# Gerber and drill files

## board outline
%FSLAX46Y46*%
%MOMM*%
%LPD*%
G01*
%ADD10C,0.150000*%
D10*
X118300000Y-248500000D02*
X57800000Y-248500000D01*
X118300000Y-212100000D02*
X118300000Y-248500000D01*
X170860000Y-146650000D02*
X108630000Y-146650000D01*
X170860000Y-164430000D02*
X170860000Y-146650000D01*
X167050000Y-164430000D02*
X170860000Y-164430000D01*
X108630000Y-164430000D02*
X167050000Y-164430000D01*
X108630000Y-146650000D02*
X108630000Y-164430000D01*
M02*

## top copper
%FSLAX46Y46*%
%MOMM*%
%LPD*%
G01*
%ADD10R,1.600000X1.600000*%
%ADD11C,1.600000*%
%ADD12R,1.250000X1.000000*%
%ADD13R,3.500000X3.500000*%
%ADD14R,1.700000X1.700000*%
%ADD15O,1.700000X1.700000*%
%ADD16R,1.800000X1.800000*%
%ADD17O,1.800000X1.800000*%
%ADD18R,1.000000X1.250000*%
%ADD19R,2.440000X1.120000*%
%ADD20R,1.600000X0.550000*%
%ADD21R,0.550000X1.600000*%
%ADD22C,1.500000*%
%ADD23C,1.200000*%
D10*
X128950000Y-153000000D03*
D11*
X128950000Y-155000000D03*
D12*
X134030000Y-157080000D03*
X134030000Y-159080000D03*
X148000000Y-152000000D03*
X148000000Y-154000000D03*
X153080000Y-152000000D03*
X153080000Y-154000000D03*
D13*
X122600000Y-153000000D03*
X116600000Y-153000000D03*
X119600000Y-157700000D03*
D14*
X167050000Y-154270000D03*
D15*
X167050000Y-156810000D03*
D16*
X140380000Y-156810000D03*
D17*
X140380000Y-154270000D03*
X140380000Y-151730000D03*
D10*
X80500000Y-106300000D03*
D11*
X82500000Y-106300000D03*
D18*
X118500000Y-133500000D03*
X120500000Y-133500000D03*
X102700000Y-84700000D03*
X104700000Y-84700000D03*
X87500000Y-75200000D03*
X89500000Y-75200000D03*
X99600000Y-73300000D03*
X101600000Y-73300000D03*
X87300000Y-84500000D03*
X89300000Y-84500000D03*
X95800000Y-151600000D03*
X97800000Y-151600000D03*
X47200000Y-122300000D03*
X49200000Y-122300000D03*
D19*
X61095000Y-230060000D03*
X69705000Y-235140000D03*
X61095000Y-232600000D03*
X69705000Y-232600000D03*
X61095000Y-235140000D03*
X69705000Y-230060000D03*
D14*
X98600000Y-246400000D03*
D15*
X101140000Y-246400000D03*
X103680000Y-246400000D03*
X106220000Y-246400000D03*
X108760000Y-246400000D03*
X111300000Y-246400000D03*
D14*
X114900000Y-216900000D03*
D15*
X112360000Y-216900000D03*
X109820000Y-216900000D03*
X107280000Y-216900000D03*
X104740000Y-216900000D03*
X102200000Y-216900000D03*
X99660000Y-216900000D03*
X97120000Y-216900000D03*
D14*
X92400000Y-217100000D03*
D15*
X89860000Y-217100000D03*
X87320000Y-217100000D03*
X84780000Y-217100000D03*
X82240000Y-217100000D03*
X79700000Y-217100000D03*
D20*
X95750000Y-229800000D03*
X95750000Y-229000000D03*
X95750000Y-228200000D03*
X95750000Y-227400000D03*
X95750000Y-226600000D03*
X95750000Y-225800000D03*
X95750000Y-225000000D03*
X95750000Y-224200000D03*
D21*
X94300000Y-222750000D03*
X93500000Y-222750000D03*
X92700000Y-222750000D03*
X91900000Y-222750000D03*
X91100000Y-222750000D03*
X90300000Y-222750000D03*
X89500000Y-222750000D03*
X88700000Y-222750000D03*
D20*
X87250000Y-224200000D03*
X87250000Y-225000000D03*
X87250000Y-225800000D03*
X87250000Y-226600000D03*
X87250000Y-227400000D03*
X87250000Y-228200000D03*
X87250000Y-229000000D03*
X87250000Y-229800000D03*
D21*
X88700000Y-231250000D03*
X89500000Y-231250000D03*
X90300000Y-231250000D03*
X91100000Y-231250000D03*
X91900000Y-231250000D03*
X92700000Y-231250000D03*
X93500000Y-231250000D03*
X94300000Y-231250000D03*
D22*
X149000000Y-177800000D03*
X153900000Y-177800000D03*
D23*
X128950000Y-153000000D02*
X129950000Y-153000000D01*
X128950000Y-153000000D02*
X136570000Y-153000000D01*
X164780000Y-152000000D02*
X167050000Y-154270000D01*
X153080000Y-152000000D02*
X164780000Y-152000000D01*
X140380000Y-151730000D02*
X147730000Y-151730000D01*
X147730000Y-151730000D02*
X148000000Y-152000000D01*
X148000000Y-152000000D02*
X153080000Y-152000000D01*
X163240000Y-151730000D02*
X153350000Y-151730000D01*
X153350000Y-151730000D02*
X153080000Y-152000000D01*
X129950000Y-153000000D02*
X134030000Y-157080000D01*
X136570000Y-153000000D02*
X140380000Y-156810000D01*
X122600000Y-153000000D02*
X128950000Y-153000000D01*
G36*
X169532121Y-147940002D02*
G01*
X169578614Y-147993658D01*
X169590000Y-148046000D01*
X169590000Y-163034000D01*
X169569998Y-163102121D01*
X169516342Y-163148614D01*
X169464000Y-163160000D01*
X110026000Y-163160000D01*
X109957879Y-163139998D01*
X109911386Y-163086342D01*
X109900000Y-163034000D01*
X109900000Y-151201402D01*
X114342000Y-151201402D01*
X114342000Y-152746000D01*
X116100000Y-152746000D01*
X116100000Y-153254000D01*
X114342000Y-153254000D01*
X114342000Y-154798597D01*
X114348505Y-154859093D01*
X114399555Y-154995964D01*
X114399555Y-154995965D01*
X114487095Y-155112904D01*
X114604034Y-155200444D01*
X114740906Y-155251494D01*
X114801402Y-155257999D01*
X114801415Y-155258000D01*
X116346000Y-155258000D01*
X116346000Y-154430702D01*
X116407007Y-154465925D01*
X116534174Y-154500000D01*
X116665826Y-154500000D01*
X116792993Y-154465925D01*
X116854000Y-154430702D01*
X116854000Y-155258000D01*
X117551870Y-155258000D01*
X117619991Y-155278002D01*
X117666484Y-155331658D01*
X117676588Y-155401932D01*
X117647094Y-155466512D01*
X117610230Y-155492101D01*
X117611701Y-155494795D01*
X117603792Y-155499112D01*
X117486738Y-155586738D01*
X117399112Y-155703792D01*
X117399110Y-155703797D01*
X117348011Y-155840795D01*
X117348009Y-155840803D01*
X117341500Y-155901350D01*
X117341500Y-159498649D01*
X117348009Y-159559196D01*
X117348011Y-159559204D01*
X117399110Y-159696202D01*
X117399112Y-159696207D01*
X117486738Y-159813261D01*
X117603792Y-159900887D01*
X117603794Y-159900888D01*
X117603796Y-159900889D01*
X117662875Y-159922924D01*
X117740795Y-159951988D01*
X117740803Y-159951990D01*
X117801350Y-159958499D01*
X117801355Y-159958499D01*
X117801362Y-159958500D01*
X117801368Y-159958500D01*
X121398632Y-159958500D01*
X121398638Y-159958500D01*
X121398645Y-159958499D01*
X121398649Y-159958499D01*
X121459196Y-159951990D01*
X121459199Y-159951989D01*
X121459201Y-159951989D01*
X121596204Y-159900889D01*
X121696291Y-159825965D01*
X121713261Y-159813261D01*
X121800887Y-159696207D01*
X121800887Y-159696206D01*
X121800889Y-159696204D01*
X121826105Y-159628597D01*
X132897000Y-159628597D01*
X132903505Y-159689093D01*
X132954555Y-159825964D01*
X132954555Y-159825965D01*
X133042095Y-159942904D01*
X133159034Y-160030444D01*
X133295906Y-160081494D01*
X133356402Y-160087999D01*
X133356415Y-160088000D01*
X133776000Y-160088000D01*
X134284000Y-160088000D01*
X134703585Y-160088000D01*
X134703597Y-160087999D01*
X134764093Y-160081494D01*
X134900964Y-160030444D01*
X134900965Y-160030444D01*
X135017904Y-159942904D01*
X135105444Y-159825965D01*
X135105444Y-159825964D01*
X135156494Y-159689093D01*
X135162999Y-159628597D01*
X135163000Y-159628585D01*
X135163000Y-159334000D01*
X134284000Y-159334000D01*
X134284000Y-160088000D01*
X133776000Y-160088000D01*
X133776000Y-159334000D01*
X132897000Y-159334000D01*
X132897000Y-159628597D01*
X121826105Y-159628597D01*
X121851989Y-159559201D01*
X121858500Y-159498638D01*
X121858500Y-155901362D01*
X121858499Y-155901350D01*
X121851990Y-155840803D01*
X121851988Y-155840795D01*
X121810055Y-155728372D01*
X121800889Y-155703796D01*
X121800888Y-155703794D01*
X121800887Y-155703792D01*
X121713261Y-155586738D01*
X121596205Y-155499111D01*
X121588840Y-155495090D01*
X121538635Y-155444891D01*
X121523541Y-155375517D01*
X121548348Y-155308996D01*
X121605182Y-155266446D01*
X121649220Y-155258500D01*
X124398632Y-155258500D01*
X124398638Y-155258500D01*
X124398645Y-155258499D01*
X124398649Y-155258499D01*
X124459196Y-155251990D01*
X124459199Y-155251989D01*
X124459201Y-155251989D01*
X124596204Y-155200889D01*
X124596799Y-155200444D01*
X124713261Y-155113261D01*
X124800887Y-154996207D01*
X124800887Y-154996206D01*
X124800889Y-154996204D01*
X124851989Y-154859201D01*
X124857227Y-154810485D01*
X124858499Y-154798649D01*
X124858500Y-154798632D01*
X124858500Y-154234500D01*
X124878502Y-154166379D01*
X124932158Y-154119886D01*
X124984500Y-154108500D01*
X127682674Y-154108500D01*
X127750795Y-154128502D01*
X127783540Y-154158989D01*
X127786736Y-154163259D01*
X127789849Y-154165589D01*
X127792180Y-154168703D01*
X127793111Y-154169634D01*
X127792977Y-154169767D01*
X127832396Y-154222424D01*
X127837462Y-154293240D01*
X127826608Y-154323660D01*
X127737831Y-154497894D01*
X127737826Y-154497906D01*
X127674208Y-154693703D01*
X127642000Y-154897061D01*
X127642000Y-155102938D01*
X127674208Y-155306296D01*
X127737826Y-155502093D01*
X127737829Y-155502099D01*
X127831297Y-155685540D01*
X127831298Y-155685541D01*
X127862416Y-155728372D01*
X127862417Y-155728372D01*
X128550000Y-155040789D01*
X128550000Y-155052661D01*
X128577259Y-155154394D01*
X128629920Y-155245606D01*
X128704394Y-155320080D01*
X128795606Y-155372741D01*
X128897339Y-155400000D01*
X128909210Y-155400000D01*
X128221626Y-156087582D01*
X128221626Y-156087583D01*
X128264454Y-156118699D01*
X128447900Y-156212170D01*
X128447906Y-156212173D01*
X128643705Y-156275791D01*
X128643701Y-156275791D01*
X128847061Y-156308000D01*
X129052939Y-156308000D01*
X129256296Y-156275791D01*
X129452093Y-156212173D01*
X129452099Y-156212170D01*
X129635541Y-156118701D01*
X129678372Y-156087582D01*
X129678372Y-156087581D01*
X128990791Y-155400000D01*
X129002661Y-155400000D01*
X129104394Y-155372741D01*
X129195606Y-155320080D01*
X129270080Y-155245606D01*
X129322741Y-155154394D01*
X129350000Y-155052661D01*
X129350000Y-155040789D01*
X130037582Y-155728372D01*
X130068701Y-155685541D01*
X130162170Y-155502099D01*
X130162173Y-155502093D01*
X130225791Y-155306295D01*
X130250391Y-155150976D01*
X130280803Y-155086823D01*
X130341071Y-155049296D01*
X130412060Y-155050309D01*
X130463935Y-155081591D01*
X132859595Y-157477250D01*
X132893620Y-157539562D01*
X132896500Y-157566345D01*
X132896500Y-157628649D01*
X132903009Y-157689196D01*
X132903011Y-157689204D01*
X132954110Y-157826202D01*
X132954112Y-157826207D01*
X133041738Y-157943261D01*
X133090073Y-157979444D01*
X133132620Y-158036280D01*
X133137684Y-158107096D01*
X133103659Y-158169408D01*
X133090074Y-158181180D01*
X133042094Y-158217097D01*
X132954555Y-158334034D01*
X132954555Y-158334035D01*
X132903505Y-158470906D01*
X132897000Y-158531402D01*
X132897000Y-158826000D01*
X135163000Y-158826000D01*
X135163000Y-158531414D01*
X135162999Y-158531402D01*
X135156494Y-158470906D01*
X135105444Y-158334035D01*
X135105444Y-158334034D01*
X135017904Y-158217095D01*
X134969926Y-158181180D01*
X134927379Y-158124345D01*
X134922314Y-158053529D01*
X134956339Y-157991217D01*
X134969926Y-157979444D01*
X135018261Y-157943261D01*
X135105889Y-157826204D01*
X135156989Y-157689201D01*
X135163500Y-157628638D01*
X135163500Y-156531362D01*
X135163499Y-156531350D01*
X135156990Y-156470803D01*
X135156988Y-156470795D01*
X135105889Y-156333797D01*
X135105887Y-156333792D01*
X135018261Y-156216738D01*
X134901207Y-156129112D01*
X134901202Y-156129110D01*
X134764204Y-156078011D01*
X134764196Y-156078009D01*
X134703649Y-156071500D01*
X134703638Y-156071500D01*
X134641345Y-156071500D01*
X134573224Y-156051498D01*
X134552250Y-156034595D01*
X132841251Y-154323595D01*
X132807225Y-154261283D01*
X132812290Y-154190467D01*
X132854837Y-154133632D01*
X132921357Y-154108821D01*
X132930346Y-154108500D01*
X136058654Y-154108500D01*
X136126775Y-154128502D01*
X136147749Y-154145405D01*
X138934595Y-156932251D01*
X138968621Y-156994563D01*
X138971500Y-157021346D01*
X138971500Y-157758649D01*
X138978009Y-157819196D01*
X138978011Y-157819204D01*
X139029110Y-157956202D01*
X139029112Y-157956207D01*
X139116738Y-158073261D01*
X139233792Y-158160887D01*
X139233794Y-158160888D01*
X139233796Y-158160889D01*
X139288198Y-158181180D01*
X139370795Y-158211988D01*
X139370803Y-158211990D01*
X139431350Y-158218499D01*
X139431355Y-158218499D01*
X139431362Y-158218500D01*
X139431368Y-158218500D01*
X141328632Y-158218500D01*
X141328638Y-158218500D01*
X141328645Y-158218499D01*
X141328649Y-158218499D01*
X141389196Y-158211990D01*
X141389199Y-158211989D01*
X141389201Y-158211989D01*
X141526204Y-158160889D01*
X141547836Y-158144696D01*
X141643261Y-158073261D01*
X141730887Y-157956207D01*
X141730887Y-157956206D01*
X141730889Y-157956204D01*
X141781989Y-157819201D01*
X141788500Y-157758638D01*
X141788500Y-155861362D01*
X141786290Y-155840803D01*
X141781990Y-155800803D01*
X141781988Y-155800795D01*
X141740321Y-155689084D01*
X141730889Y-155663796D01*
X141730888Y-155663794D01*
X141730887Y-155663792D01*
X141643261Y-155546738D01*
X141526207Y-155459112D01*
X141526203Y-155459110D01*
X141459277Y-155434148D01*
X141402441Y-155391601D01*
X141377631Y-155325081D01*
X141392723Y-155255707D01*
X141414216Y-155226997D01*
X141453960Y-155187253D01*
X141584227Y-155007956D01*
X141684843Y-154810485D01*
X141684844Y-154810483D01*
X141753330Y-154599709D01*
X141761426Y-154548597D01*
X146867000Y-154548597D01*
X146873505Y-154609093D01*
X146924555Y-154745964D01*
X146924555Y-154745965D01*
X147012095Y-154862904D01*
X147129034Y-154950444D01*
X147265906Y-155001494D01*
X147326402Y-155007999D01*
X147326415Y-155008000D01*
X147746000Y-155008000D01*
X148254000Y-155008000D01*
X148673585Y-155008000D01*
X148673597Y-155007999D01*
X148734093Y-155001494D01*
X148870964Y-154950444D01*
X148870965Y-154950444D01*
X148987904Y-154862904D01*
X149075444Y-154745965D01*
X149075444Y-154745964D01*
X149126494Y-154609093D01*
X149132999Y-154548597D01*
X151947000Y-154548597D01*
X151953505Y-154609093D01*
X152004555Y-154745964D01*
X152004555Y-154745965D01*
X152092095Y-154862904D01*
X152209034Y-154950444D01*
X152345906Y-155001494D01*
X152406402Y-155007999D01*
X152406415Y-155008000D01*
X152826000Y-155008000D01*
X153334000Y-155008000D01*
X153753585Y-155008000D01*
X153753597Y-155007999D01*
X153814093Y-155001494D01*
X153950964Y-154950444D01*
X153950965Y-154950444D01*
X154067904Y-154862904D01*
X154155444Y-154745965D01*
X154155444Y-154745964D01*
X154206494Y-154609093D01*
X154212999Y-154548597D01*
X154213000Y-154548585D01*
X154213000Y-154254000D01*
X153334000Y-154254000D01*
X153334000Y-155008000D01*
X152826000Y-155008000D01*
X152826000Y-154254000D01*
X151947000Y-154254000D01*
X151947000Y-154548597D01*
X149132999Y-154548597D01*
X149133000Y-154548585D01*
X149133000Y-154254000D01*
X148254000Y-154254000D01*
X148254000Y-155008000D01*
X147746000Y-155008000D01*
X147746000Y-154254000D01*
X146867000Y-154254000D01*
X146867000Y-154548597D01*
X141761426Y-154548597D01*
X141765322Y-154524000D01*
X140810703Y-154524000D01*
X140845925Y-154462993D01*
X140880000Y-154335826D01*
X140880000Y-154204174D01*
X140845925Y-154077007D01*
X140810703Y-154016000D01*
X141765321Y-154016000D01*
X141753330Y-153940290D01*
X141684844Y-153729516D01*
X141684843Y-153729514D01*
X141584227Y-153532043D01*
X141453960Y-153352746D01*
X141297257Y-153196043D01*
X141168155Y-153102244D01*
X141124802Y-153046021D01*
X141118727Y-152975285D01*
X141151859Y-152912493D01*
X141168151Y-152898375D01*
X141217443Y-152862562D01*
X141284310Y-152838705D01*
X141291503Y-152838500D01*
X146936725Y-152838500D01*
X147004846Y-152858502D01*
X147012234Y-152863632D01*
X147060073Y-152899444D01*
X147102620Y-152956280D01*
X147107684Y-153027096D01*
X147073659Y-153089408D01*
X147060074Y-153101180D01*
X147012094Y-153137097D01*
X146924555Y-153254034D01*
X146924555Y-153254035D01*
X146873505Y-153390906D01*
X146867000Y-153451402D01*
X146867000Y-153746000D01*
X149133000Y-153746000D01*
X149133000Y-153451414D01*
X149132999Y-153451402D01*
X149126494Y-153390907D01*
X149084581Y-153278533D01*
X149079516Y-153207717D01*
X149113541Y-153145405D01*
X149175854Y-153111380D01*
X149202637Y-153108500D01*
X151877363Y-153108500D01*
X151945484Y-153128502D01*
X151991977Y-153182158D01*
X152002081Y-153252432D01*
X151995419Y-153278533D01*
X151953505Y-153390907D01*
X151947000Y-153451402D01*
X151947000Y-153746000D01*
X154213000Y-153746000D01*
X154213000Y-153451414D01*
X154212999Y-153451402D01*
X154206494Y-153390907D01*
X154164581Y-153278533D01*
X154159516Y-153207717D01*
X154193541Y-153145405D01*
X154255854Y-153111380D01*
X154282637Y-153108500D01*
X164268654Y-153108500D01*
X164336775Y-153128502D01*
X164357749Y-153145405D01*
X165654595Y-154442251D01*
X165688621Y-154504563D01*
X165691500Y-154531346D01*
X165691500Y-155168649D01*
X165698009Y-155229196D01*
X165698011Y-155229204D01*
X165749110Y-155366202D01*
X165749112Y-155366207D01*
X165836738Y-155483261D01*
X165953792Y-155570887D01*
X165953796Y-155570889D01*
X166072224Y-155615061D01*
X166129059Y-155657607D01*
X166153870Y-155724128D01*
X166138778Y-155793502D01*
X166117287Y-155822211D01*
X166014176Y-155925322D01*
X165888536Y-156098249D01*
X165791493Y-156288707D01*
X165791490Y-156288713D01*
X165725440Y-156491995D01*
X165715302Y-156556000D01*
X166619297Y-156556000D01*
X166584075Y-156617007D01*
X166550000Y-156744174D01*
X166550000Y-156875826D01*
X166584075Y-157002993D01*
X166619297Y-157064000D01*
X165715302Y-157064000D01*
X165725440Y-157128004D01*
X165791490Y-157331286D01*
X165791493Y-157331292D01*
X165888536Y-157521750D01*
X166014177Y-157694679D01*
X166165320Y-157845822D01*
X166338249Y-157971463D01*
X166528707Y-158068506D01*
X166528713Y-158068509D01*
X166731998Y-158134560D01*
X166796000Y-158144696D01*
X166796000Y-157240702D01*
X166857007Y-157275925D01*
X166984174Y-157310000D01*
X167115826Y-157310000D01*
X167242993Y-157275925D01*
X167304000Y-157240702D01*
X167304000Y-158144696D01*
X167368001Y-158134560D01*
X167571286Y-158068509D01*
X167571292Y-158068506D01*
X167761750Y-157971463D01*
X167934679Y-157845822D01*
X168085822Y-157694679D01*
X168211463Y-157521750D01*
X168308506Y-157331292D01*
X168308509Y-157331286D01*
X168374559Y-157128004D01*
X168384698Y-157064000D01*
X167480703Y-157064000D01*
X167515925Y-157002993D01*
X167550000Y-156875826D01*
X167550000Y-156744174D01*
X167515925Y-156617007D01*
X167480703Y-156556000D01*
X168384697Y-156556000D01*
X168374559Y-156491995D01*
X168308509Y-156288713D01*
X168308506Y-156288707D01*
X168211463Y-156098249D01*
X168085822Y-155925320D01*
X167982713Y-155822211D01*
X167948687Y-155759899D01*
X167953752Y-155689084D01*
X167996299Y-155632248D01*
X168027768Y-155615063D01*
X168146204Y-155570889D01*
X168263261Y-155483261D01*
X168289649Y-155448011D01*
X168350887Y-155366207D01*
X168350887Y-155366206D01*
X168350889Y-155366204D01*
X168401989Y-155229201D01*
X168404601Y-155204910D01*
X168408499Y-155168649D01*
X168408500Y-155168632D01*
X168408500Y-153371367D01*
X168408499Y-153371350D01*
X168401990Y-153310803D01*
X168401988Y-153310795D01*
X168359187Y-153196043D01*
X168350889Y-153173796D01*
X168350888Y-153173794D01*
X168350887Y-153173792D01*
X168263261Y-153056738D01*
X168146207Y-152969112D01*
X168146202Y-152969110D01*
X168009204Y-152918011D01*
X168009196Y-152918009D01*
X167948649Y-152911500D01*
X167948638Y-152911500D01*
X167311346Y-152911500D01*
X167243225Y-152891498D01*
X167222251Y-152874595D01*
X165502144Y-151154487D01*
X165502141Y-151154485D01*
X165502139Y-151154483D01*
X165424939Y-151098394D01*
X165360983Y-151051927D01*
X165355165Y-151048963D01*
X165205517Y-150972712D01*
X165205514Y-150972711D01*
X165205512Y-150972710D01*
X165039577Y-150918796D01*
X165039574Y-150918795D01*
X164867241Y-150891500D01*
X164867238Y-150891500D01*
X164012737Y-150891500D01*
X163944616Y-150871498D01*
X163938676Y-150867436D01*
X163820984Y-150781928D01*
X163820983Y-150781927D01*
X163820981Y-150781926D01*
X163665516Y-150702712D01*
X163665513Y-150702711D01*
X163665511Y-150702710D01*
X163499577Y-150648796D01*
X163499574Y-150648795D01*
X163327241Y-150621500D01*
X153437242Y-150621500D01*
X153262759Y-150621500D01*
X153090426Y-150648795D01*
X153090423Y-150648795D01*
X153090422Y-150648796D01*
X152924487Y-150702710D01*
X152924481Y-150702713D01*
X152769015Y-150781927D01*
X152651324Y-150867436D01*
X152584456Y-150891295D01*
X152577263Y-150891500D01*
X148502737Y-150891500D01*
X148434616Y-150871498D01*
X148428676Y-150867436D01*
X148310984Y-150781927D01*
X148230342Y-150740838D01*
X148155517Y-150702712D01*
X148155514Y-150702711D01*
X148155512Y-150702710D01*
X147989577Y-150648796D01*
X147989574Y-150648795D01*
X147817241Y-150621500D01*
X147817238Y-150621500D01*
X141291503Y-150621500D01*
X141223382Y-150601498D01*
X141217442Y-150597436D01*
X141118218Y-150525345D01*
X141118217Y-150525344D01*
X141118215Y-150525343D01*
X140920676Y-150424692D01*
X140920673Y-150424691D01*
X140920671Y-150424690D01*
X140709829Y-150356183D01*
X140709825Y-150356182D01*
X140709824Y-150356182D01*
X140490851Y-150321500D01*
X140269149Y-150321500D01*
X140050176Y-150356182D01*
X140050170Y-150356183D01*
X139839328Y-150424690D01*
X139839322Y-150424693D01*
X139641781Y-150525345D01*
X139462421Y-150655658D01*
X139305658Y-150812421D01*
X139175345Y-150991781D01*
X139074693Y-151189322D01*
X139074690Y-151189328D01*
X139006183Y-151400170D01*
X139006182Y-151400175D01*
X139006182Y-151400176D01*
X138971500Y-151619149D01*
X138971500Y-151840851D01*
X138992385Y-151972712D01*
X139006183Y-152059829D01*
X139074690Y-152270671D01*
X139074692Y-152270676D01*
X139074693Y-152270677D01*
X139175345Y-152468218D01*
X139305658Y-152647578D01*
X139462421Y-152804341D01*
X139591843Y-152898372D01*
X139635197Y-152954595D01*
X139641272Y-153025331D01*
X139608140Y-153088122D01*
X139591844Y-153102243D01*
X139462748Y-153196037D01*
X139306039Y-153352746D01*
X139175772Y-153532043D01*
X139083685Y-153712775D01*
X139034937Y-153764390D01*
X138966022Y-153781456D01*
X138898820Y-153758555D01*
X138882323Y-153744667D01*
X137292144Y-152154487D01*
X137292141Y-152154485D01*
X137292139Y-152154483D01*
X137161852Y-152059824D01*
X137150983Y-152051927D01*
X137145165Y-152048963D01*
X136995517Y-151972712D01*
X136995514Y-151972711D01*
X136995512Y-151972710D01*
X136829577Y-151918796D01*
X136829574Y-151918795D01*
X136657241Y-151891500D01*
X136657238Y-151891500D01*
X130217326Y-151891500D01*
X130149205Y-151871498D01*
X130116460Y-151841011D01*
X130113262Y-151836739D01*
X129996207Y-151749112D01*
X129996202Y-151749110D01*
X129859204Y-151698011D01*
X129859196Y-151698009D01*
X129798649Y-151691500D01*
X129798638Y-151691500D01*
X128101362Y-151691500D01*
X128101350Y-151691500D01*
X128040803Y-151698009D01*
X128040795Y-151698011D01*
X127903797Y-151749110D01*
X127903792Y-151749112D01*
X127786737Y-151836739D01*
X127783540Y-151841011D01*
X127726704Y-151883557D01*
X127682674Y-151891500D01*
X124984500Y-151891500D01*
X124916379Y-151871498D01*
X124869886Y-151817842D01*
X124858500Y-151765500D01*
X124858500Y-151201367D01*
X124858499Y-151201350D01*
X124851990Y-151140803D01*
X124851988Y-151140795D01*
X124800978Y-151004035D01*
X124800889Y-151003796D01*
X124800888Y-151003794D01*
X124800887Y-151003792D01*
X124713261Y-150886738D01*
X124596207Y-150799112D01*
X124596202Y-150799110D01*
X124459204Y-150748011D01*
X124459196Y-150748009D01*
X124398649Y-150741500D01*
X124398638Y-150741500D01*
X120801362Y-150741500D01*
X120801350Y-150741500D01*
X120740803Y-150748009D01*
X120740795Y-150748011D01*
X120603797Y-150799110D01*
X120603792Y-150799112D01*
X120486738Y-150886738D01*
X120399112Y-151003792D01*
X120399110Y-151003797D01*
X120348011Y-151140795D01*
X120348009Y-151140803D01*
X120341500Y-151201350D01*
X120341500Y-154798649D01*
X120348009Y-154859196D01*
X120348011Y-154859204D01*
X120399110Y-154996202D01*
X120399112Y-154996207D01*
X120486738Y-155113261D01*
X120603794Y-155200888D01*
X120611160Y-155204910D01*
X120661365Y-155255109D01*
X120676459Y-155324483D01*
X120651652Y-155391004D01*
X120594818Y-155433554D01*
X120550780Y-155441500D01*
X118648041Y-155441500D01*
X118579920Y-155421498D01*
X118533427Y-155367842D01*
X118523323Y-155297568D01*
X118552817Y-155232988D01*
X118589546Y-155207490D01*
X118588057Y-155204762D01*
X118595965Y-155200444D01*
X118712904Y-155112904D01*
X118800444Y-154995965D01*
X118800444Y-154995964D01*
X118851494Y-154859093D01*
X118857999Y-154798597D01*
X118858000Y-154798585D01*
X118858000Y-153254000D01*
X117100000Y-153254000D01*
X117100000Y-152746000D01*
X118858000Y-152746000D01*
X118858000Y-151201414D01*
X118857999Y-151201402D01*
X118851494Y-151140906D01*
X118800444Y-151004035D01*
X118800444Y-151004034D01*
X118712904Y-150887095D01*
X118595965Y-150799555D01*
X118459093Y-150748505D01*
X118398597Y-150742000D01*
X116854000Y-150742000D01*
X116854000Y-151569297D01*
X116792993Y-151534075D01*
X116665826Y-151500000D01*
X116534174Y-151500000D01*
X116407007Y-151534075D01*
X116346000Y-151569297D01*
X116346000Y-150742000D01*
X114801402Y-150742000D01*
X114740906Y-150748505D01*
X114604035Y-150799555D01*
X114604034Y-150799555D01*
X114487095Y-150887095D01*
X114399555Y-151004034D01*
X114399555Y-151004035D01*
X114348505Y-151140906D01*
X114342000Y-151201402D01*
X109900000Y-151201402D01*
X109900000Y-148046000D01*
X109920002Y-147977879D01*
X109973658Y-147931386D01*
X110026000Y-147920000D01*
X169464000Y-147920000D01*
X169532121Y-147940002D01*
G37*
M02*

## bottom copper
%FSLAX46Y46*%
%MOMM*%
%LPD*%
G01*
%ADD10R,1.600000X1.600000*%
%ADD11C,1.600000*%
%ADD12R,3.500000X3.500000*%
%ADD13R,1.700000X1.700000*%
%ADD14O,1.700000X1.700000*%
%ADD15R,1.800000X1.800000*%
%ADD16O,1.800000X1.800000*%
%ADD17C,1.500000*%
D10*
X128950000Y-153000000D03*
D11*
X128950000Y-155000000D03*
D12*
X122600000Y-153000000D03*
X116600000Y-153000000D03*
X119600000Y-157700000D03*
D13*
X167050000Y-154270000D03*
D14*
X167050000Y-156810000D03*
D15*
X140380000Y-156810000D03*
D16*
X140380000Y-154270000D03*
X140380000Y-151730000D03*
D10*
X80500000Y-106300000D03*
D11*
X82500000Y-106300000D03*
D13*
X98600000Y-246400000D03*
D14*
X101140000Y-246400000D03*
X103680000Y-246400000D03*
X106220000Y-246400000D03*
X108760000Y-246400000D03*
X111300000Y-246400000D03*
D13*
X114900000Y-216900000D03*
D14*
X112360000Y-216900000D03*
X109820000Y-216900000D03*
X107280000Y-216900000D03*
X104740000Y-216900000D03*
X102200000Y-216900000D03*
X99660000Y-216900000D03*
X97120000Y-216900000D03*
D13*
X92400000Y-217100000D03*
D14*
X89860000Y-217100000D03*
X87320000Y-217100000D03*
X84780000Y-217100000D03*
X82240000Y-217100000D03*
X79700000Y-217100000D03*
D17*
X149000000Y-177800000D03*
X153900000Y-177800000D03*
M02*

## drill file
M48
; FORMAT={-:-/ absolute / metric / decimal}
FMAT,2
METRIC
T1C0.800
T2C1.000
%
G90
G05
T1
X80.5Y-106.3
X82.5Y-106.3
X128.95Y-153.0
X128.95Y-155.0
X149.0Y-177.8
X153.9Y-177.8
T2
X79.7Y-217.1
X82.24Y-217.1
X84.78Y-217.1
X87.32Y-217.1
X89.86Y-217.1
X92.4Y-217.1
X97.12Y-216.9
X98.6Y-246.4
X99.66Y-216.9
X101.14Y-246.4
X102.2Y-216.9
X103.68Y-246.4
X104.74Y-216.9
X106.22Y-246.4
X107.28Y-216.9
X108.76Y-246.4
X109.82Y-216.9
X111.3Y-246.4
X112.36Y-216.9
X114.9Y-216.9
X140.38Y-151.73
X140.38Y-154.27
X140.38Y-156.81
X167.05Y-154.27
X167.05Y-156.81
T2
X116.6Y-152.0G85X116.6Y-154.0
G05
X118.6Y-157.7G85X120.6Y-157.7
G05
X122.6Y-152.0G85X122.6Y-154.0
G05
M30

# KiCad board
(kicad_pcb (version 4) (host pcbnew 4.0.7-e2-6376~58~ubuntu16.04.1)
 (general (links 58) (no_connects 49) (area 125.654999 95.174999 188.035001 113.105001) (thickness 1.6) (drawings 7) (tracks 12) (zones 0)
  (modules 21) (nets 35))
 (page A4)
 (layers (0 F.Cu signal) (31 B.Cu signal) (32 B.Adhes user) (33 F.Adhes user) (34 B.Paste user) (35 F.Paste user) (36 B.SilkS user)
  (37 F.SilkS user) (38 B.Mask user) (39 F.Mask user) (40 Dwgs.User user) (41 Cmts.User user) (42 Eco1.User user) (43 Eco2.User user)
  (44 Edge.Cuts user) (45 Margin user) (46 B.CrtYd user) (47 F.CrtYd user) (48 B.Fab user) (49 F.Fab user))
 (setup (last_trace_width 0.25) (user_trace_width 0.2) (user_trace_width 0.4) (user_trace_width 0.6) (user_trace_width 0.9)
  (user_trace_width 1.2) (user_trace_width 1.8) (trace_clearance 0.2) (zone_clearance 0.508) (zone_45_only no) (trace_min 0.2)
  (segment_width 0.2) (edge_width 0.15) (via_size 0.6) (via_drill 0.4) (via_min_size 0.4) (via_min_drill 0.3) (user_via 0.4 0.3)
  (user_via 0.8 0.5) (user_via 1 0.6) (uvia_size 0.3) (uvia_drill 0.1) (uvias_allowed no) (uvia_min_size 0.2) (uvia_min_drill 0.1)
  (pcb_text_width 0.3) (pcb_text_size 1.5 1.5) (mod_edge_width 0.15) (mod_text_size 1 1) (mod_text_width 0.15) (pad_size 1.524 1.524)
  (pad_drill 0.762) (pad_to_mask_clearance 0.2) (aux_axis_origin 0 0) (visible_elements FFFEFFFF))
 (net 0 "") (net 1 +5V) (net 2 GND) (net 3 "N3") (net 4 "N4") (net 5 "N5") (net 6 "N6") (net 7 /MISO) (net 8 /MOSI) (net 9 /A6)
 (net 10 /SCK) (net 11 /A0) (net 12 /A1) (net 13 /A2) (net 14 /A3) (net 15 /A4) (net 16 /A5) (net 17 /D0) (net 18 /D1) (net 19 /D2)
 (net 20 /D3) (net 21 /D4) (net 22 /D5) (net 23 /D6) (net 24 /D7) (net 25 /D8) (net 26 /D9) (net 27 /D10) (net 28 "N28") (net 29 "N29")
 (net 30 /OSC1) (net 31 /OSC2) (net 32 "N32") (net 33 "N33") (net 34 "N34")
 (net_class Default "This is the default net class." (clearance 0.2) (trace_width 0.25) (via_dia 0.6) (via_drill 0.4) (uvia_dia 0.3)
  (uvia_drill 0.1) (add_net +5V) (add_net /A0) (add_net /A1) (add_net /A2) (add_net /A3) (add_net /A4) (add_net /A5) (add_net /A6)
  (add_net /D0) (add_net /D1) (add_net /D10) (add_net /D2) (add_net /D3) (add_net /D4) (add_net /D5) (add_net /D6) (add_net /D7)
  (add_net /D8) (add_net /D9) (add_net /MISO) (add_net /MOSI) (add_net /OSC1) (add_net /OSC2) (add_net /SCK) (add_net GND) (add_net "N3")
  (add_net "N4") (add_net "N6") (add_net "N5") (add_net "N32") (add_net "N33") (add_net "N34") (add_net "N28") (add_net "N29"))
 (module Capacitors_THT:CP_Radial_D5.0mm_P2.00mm (layer F.Cu) (at 128.95 153 270)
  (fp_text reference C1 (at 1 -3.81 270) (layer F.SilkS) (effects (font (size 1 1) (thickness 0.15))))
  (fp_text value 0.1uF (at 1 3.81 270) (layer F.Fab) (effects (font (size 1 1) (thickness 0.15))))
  (pad 1 thru_hole rect (at 0 0 270) (size 1.6 1.6) (drill 0.8) (layers *.Cu *.Mask) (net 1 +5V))
  (pad 2 thru_hole circle (at 2 0 270) (size 1.6 1.6) (drill 0.8) (layers *.Cu *.Mask) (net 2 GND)))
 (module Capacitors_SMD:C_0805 (layer F.Cu) (at 134.03 158.08 270)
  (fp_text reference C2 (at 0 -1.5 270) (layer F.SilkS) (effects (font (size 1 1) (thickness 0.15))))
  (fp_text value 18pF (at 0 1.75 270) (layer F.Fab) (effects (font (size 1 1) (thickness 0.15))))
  (pad 1 smd rect (at -1 0 270) (size 1 1.25) (layers F.Cu F.Paste F.Mask) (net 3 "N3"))
  (pad 2 smd rect (at 1 0 270) (size 1 1.25) (layers F.Cu F.Paste F.Mask) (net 2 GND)))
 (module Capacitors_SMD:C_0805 (layer F.Cu) (at 148 153 270)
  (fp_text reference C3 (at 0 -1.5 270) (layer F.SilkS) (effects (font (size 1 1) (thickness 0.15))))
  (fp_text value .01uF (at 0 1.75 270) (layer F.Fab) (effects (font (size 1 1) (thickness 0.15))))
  (pad 1 smd rect (at -1 0 270) (size 1 1.25) (layers F.Cu F.Paste F.Mask) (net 1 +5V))
  (pad 2 smd rect (at 1 0 270) (size 1 1.25) (layers F.Cu F.Paste F.Mask) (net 2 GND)))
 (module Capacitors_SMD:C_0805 (layer F.Cu) (at 153.08 153 270)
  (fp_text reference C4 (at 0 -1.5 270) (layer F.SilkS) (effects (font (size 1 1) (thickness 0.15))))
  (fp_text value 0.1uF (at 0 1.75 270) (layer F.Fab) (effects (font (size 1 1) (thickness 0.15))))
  (pad 1 smd rect (at -1 0 270) (size 1 1.25) (layers F.Cu F.Paste F.Mask) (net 1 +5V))
  (pad 2 smd rect (at 1 0 270) (size 1 1.25) (layers F.Cu F.Paste F.Mask) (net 2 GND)))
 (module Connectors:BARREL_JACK (layer F.Cu) (at 122.6 153)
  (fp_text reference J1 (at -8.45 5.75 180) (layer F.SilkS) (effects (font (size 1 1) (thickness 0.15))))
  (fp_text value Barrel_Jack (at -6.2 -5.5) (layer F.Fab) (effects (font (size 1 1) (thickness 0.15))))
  (pad 1 thru_hole rect (at 0 0) (size 3.5 3.5) (drill oval 1 3) (layers *.Cu *.Mask) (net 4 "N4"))
  (pad 2 thru_hole rect (at -6 0) (size 3.5 3.5) (drill oval 1 3) (layers *.Cu *.Mask) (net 2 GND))
  (pad 3 thru_hole rect (at -3 4.7) (size 3.5 3.5) (drill oval 3 1) (layers *.Cu *.Mask) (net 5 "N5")))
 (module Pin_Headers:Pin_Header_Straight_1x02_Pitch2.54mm (layer F.Cu) (at 167.05 154.27)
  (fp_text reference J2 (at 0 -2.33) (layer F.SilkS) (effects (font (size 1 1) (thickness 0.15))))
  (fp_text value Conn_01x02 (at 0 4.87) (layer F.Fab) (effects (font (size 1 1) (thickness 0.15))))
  (pad 1 thru_hole rect (at 0 0) (size 1.7 1.7) (drill 1) (layers *.Cu *.Mask) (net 1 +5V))
  (pad 2 thru_hole oval (at 0 2.54) (size 1.7 1.7) (drill 1) (layers *.Cu *.Mask) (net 2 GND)))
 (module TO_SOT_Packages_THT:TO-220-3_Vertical (layer F.Cu) (at 140.38 156.81 90)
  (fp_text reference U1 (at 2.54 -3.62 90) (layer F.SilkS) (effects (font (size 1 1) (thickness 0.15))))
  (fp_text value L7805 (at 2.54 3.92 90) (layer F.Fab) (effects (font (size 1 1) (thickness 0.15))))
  (pad 1 thru_hole rect (at 0 0 90) (size 1.8 1.8) (drill 1) (layers *.Cu *.Mask) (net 4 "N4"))
  (pad 2 thru_hole oval (at 2.54 0 90) (size 1.8 1.8) (drill 1) (layers *.Cu *.Mask) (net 2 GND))
  (pad 3 thru_hole oval (at 5.08 0 90) (size 1.8 1.8) (drill 1) (layers *.Cu *.Mask) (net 1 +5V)))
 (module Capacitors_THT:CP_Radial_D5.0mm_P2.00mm (layer F.Cu) (at 80.5 106.3)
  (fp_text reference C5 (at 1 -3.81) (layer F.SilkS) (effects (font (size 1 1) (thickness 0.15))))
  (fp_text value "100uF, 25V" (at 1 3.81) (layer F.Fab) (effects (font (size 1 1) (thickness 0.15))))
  (pad 1 thru_hole rect (at 0 0) (size 1.6 1.6) (drill 0.8) (layers *.Cu *.Mask) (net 4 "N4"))
  (pad 2 thru_hole circle (at 2 0) (size 1.6 1.6) (drill 0.8) (layers *.Cu *.Mask) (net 2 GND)))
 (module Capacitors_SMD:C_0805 (layer F.Cu) (at 119.5 133.5)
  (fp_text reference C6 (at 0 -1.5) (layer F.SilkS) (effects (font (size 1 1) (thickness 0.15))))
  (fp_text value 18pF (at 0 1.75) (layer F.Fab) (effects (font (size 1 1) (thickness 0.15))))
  (pad 1 smd rect (at -1 0) (size 1 1.25) (layers F.Cu F.Paste F.Mask) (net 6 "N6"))
  (pad 2 smd rect (at 1 0) (size 1 1.25) (layers F.Cu F.Paste F.Mask) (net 2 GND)))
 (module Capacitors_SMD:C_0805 (layer F.Cu) (at 103.7 84.7)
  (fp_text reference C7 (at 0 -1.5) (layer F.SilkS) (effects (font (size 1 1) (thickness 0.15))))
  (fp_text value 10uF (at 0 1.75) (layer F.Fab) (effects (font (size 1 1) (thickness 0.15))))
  (pad 1 smd rect (at -1 0) (size 1 1.25) (layers F.Cu F.Paste F.Mask) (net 4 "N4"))
  (pad 2 smd rect (at 1 0) (size 1 1.25) (layers F.Cu F.Paste F.Mask) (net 2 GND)))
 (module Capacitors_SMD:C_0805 (layer F.Cu) (at 88.5 75.2)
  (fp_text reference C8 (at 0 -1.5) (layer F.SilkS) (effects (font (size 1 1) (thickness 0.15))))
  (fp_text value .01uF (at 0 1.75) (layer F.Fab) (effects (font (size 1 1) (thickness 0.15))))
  (pad 1 smd rect (at -1 0) (size 1 1.25) (layers F.Cu F.Paste F.Mask) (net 1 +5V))
  (pad 2 smd rect (at 1 0) (size 1 1.25) (layers F.Cu F.Paste F.Mask) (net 2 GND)))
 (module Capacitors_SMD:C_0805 (layer F.Cu) (at 100.6 73.3)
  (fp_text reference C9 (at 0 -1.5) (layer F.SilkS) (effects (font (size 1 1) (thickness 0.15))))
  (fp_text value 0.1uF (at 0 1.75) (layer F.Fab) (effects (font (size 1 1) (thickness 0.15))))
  (pad 1 smd rect (at -1 0) (size 1 1.25) (layers F.Cu F.Paste F.Mask) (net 1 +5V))
  (pad 2 smd rect (at 1 0) (size 1 1.25) (layers F.Cu F.Paste F.Mask) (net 2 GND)))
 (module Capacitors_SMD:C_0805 (layer F.Cu) (at 88.3 84.5)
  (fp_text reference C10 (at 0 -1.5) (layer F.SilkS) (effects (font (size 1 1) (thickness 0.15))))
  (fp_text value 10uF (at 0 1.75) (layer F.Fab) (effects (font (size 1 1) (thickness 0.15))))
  (pad 1 smd rect (at -1 0) (size 1 1.25) (layers F.Cu F.Paste F.Mask) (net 1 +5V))
  (pad 2 smd rect (at 1 0) (size 1 1.25) (layers F.Cu F.Paste F.Mask) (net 2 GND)))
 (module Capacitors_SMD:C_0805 (layer F.Cu) (at 96.8 151.6)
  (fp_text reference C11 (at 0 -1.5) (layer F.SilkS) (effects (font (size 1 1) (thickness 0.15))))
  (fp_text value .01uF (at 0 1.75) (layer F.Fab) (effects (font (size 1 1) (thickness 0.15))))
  (pad 1 smd rect (at -1 0) (size 1 1.25) (layers F.Cu F.Paste F.Mask) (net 1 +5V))
  (pad 2 smd rect (at 1 0) (size 1 1.25) (layers F.Cu F.Paste F.Mask) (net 2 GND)))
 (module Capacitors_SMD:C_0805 (layer F.Cu) (at 48.2 122.3)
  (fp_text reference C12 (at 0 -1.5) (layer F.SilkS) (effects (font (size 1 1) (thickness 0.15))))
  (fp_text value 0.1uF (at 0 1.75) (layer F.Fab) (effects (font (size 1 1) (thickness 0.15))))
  (pad 1 smd rect (at -1 0) (size 1 1.25) (layers F.Cu F.Paste F.Mask) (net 1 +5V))
  (pad 2 smd rect (at 1 0) (size 1 1.25) (layers F.Cu F.Paste F.Mask) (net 2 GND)))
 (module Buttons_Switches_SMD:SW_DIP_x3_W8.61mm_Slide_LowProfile (layer F.Cu) (at 65.4 232.6)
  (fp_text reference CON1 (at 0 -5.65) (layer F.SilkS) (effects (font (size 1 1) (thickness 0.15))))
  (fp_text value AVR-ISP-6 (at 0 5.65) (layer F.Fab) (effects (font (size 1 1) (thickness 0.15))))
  (pad 1 smd rect (at -4.305 -2.54) (size 2.44 1.12) (layers F.Cu F.Paste F.Mask) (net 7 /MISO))
  (pad 4 smd rect (at 4.305 2.54) (size 2.44 1.12) (layers F.Cu F.Paste F.Mask) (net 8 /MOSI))
  (pad 2 smd rect (at -4.305 0) (size 2.44 1.12) (layers F.Cu F.Paste F.Mask) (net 1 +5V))
  (pad 5 smd rect (at 4.305 0) (size 2.44 1.12) (layers F.Cu F.Paste F.Mask) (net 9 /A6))
  (pad 3 smd rect (at -4.305 2.54) (size 2.44 1.12) (layers F.Cu F.Paste F.Mask) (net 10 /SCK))
  (pad 6 smd rect (at 4.305 -2.54) (size 2.44 1.12) (layers F.Cu F.Paste F.Mask) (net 2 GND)))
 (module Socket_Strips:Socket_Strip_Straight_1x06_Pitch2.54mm (layer F.Cu) (at 98.6 246.4 90)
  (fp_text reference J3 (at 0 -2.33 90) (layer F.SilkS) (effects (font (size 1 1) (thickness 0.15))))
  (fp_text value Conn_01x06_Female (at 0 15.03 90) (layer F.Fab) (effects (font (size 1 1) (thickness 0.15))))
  (pad 1 thru_hole rect (at 0 0 90) (size 1.7 1.7) (drill 1) (layers *.Cu *.Mask) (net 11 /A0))
  (pad 2 thru_hole oval (at 0 2.54 90) (size 1.7 1.7) (drill 1) (layers *.Cu *.Mask) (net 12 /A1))
  (pad 3 thru_hole oval (at 0 5.08 90) (size 1.7 1.7) (drill 1) (layers *.Cu *.Mask) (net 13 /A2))
  (pad 4 thru_hole oval (at 0 7.62 90) (size 1.7 1.7) (drill 1) (layers *.Cu *.Mask) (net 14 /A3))
  (pad 5 thru_hole oval (at 0 10.16 90) (size 1.7 1.7) (drill 1) (layers *.Cu *.Mask) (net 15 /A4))
  (pad 6 thru_hole oval (at 0 12.7 90) (size 1.7 1.7) (drill 1) (layers *.Cu *.Mask) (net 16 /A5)))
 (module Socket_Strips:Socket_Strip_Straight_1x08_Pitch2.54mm (layer F.Cu) (at 114.9 216.9 270)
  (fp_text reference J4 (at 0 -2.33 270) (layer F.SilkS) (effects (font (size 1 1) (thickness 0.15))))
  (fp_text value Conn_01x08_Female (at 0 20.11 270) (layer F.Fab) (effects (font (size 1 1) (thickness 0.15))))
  (pad 1 thru_hole rect (at 0 0 270) (size 1.7 1.7) (drill 1) (layers *.Cu *.Mask) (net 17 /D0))
  (pad 2 thru_hole oval (at 0 2.54 270) (size 1.7 1.7) (drill 1) (layers *.Cu *.Mask) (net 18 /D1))
  (pad 3 thru_hole oval (at 0 5.08 270) (size 1.7 1.7) (drill 1) (layers *.Cu *.Mask) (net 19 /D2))
  (pad 4 thru_hole oval (at 0 7.62 270) (size 1.7 1.7) (drill 1) (layers *.Cu *.Mask) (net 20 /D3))
  (pad 5 thru_hole oval (at 0 10.16 270) (size 1.7 1.7) (drill 1) (layers *.Cu *.Mask) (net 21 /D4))
  (pad 6 thru_hole oval (at 0 12.7 270) (size 1.7 1.7) (drill 1) (layers *.Cu *.Mask) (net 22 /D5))
  (pad 7 thru_hole oval (at 0 15.24 270) (size 1.7 1.7) (drill 1) (layers *.Cu *.Mask) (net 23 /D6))
  (pad 8 thru_hole oval (at 0 17.78 270) (size 1.7 1.7) (drill 1) (layers *.Cu *.Mask) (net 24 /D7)))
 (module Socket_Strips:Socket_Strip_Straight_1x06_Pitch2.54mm (layer B.Cu) (at 92.4 217.1 90)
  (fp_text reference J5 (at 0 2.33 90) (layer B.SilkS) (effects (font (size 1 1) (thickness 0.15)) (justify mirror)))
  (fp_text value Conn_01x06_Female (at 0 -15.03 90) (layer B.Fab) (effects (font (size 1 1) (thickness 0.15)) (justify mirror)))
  (pad 1 thru_hole rect (at 0 0 90) (size 1.7 1.7) (drill 1) (layers *.Cu *.Mask) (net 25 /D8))
  (pad 2 thru_hole oval (at 0 -2.54 90) (size 1.7 1.7) (drill 1) (layers *.Cu *.Mask) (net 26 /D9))
  (pad 3 thru_hole oval (at 0 -5.08 90) (size 1.7 1.7) (drill 1) (layers *.Cu *.Mask) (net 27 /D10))
  (pad 4 thru_hole oval (at 0 -7.62 90) (size 1.7 1.7) (drill 1) (layers *.Cu *.Mask) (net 8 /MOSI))
  (pad 5 thru_hole oval (at 0 -10.16 90) (size 1.7 1.7) (drill 1) (layers *.Cu *.Mask) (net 7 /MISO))
  (pad 6 thru_hole oval (at 0 -12.7 90) (size 1.7 1.7) (drill 1) (layers *.Cu *.Mask) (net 10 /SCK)))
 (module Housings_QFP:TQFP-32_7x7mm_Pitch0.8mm (layer F.Cu) (at 91.5 227 180)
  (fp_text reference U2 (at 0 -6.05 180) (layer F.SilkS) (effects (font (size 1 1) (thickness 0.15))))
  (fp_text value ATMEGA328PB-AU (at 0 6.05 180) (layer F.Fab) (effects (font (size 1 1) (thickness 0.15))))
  (pad 1 smd rect (at -4.25 -2.8 180) (size 1.6 0.55) (layers F.Cu F.Paste F.Mask) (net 20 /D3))
  (pad 2 smd rect (at -4.25 -2 180) (size 1.6 0.55) (layers F.Cu F.Paste F.Mask) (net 21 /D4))
  (pad 3 smd rect (at -4.25 -1.2 180) (size 1.6 0.55) (layers F.Cu F.Paste F.Mask) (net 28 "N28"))
  (pad 4 smd rect (at -4.25 -0.4 180) (size 1.6 0.55) (layers F.Cu F.Paste F.Mask) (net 1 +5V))
  (pad 5 smd rect (at -4.25 0.4 180) (size 1.6 0.55) (layers F.Cu F.Paste F.Mask) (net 2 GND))
  (pad 6 smd rect (at -4.25 1.2 180) (size 1.6 0.55) (layers F.Cu F.Paste F.Mask) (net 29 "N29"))
  (pad 7 smd rect (at -4.25 2 180) (size 1.6 0.55) (layers F.Cu F.Paste F.Mask) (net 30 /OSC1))
  (pad 8 smd rect (at -4.25 2.8 180) (size 1.6 0.55) (layers F.Cu F.Paste F.Mask) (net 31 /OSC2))
  (pad 9 smd rect (at -2.8 4.25 270) (size 1.6 0.55) (layers F.Cu F.Paste F.Mask) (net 22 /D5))
  (pad 10 smd rect (at -2 4.25 270) (size 1.6 0.55) (layers F.Cu F.Paste F.Mask) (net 23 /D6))
  (pad 11 smd rect (at -1.2 4.25 270) (size 1.6 0.55) (layers F.Cu F.Paste F.Mask) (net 24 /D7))
  (pad 12 smd rect (at -0.4 4.25 270) (size 1.6 0.55) (layers F.Cu F.Paste F.Mask) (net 25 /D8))
  (pad 13 smd rect (at 0.4 4.25 270) (size 1.6 0.55) (layers F.Cu F.Paste F.Mask) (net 26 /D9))
  (pad 14 smd rect (at 1.2 4.25 270) (size 1.6 0.55) (layers F.Cu F.Paste F.Mask) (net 27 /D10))
  (pad 15 smd rect (at 2 4.25 270) (size 1.6 0.55) (layers F.Cu F.Paste F.Mask) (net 8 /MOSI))
  (pad 16 smd rect (at 2.8 4.25 270) (size 1.6 0.55) (layers F.Cu F.Paste F.Mask) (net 7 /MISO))
  (pad 17 smd rect (at 4.25 2.8 180) (size 1.6 0.55) (layers F.Cu F.Paste F.Mask) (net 10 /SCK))
  (pad 18 smd rect (at 4.25 2 180) (size 1.6 0.55) (layers F.Cu F.Paste F.Mask) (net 1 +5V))
  (pad 19 smd rect (at 4.25 1.2 180) (size 1.6 0.55) (layers F.Cu F.Paste F.Mask) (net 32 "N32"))
  (pad 20 smd rect (at 4.25 0.4 180) (size 1.6 0.55) (layers F.Cu F.Paste F.Mask) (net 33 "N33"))
  (pad 21 smd rect (at 4.25 -0.4 180) (size 1.6 0.55) (layers F.Cu F.Paste F.Mask) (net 2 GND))
  (pad 22 smd rect (at 4.25 -1.2 180) (size 1.6 0.55) (layers F.Cu F.Paste F.Mask) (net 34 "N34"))
  (pad 23 smd rect (at 4.25 -2 180) (size 1.6 0.55) (layers F.Cu F.Paste F.Mask) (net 11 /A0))
  (pad 24 smd rect (at 4.25 -2.8 180) (size 1.6 0.55) (layers F.Cu F.Paste F.Mask) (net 12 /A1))
  (pad 25 smd rect (at 2.8 -4.25 270) (size 1.6 0.55) (layers F.Cu F.Paste F.Mask) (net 13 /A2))
  (pad 26 smd rect (at 2 -4.25 270) (size 1.6 0.55) (layers F.Cu F.Paste F.Mask) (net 14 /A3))
  (pad 27 smd rect (at 1.2 -4.25 270) (size 1.6 0.55) (layers F.Cu F.Paste F.Mask) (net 15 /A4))
  (pad 28 smd rect (at 0.4 -4.25 270) (size 1.6 0.55) (layers F.Cu F.Paste F.Mask) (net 16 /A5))
  (pad 29 smd rect (at -0.4 -4.25 270) (size 1.6 0.55) (layers F.Cu F.Paste F.Mask) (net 9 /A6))
  (pad 30 smd rect (at -1.2 -4.25 270) (size 1.6 0.55) (layers F.Cu F.Paste F.Mask) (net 17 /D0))
  (pad 31 smd rect (at -2 -4.25 270) (size 1.6 0.55) (layers F.Cu F.Paste F.Mask) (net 18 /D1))
  (pad 32 smd rect (at -2.8 -4.25 270) (size 1.6 0.55) (layers F.Cu F.Paste F.Mask) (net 19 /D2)))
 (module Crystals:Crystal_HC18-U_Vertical (layer F.Cu) (at 149 177.8)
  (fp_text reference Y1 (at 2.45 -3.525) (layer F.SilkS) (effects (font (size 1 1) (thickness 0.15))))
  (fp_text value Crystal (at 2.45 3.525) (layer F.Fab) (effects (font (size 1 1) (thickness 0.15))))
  (pad 1 thru_hole circle (at 0 0) (size 1.5 1.5) (drill 0.8) (layers *.Cu *.Mask) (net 3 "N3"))
  (pad 2 thru_hole circle (at 4.9 0) (size 1.5 1.5) (drill 0.8) (layers *.Cu *.Mask) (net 6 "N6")))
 (gr_line (start 118.3 248.5) (end 57.8 248.5) (angle 90) (layer Edge.Cuts) (width 0.15))
 (gr_line (start 118.3 212.1) (end 118.3 248.5) (angle 90) (layer Edge.Cuts) (width 0.15))
 (gr_line (start 170.86 146.65) (end 108.63 146.65) (angle 90) (layer Edge.Cuts) (width 0.15))
 (gr_line (start 170.86 164.43) (end 170.86 146.65) (angle 90) (layer Edge.Cuts) (width 0.15))
 (gr_line (start 167.05 164.43) (end 170.86 164.43) (angle 90) (layer Edge.Cuts) (width 0.15))
 (gr_line (start 108.63 164.43) (end 167.05 164.43) (angle 90) (layer Edge.Cuts) (width 0.15))
 (gr_line (start 108.63 146.65) (end 108.63 164.43) (angle 90) (layer Edge.Cuts) (width 0.15))
 (segment (start 128.95 153) (end 129.95 153) (width 1.2) (layer F.Cu) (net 1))
 (segment (start 128.95 153) (end 136.57 153) (width 1.2) (layer F.Cu) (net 1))
 (segment (start 164.78 152) (end 167.05 154.27) (width 1.2) (layer F.Cu) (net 1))
 (segment (start 153.08 152) (end 164.78 152) (width 1.2) (layer F.Cu) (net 1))
 (segment (start 140.38 151.73) (end 147.73 151.73) (width 1.2) (layer F.Cu) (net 1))
 (segment (start 147.73 151.73) (end 148 152) (width 1.2) (layer F.Cu) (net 1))
 (segment (start 148 152) (end 153.08 152) (width 1.2) (layer F.Cu) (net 1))
 (segment (start 163.24 151.73) (end 153.35 151.73) (width 1.2) (layer F.Cu) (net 1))
 (segment (start 153.35 151.73) (end 153.08 152) (width 1.2) (layer F.Cu) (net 1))
 (segment (start 129.95 153) (end 134.03 157.08) (width 1.2) (layer F.Cu) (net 3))
 (segment (start 136.57 153) (end 140.38 156.81) (width 1.2) (layer F.Cu) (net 4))
 (segment (start 122.6 153) (end 128.95 153) (width 1.2) (layer F.Cu) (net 4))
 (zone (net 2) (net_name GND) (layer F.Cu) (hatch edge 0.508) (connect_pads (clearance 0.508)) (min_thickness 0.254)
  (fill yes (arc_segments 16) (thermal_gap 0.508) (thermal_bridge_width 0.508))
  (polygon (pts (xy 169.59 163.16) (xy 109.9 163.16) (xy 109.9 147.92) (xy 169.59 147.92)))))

